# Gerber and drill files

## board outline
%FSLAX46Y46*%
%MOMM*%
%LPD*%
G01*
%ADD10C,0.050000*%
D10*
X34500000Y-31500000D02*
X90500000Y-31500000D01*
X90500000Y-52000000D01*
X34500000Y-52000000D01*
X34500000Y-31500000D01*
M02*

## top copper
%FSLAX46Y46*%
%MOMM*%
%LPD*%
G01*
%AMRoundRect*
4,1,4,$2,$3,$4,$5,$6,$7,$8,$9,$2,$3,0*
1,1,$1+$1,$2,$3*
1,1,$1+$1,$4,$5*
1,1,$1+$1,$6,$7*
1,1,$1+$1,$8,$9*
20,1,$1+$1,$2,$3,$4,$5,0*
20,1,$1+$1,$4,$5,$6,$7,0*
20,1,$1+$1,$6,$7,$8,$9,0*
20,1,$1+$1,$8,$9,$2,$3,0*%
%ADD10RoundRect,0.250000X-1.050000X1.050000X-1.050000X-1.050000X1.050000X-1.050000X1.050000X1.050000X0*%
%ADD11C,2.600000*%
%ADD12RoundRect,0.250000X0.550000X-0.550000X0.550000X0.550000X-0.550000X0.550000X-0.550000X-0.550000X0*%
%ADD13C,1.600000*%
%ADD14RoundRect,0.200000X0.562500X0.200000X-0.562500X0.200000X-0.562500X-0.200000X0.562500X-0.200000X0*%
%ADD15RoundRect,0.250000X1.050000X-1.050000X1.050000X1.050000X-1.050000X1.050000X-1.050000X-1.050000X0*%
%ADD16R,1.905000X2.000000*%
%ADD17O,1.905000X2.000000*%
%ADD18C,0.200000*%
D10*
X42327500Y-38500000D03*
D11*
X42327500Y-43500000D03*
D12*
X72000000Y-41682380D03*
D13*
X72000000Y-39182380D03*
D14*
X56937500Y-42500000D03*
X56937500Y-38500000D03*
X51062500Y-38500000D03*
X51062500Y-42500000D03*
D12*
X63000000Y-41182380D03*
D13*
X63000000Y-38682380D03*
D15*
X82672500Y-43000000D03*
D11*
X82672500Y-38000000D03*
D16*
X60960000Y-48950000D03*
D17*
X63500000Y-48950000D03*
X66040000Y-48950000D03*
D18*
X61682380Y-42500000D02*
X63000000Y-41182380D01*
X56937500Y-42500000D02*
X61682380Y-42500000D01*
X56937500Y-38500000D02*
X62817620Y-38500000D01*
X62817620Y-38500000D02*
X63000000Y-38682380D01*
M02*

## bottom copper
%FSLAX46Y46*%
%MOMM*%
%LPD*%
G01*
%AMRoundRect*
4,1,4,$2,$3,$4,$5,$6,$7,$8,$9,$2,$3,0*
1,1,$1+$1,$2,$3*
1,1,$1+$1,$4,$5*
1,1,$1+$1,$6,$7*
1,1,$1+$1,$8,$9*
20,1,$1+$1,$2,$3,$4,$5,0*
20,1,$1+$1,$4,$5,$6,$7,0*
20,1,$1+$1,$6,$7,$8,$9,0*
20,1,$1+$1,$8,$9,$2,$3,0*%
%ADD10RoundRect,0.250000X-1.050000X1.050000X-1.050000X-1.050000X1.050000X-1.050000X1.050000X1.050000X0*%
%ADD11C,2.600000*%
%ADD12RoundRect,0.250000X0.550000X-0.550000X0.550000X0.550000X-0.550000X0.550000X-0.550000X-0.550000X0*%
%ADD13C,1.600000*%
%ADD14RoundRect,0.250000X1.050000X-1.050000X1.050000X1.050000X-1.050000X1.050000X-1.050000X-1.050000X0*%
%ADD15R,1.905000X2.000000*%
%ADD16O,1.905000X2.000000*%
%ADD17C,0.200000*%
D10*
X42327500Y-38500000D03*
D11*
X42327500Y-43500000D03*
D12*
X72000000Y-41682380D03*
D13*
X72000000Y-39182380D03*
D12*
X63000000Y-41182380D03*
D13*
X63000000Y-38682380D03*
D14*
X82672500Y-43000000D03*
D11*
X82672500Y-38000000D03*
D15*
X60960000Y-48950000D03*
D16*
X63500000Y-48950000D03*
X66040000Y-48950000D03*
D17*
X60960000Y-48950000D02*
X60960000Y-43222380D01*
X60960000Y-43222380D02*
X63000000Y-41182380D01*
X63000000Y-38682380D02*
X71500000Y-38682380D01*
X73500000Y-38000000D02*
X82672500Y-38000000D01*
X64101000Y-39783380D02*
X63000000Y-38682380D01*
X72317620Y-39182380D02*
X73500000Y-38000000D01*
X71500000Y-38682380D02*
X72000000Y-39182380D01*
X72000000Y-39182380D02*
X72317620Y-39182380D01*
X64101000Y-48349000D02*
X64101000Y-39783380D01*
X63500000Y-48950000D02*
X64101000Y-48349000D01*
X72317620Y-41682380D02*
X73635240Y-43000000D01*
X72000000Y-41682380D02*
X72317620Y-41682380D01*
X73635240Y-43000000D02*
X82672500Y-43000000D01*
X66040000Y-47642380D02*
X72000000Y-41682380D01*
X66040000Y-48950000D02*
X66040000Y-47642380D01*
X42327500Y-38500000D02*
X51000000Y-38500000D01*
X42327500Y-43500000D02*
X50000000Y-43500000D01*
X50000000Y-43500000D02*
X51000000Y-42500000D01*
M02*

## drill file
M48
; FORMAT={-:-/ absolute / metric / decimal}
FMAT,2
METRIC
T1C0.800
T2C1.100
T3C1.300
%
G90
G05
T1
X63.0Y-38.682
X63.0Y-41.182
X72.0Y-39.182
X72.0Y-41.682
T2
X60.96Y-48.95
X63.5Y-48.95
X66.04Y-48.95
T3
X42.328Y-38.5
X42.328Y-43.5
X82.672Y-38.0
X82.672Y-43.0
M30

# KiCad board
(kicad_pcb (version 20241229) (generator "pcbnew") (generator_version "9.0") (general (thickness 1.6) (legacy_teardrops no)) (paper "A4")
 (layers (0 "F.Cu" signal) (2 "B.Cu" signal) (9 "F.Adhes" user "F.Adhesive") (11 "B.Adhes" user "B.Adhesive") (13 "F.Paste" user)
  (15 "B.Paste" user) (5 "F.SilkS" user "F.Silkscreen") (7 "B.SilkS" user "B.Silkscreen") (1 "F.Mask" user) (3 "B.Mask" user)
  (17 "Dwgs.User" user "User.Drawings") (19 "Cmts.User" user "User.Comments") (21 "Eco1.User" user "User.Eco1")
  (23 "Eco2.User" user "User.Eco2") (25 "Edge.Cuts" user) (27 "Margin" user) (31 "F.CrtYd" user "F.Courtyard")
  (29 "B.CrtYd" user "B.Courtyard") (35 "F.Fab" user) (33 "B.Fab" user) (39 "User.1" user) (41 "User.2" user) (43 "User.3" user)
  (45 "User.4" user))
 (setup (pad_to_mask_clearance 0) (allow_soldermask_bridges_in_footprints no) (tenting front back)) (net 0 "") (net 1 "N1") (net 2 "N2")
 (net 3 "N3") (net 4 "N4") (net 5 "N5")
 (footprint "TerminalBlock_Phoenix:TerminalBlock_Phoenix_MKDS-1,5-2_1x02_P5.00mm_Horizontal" (layer "F.Cu") (at 42.3275 38.5 -90)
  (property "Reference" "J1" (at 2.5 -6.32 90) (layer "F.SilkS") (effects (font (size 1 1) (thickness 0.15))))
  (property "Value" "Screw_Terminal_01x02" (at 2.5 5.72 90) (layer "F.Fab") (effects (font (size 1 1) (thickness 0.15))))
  (pad "1" thru_hole roundrect (at 0 0 270) (size 2.6 2.6) (drill 1.3) (layers "*.Cu" "*.Mask") (remove_unused_layers no)
   (roundrect_rratio 0.096154) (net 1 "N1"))
  (pad "2" thru_hole circle (at 5 0 270) (size 2.6 2.6) (drill 1.3) (layers "*.Cu" "*.Mask") (remove_unused_layers no) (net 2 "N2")))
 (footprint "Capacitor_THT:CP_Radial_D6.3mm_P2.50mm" (layer "F.Cu") (at 72 41.68238 90)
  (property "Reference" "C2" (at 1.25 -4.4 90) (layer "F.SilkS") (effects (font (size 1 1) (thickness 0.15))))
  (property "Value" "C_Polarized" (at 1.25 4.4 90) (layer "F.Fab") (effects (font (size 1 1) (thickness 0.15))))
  (pad "1" thru_hole roundrect (at 0 0 90) (size 1.6 1.6) (drill 0.8) (layers "*.Cu" "*.Mask") (remove_unused_layers no)
   (roundrect_rratio 0.15625) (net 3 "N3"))
  (pad "2" thru_hole circle (at 2.5 0 90) (size 1.6 1.6) (drill 0.8) (layers "*.Cu" "*.Mask") (remove_unused_layers no) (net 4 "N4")))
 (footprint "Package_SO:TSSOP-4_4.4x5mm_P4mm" (layer "F.Cu") (at 54 40.5 180)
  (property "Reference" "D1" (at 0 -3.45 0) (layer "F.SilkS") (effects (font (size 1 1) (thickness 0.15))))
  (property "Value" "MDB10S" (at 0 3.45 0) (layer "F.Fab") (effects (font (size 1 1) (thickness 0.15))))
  (pad "1" smd roundrect (at -2.9375 -2 180) (size 1.525 0.8) (layers "F.Cu" "F.Mask" "F.Paste") (roundrect_rratio 0.25) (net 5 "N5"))
  (pad "2" smd roundrect (at -2.9375 2 180) (size 1.525 0.8) (layers "F.Cu" "F.Mask" "F.Paste") (roundrect_rratio 0.25) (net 4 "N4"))
  (pad "3" smd roundrect (at 2.9375 2 180) (size 1.525 0.8) (layers "F.Cu" "F.Mask" "F.Paste") (roundrect_rratio 0.25) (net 1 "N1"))
  (pad "4" smd roundrect (at 2.9375 -2 180) (size 1.525 0.8) (layers "F.Cu" "F.Mask" "F.Paste") (roundrect_rratio 0.25) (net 2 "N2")))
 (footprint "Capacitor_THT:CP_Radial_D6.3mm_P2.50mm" (layer "F.Cu") (at 63 41.18238 90)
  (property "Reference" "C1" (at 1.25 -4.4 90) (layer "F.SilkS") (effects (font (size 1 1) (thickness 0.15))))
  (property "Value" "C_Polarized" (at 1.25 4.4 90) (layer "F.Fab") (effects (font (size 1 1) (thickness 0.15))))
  (pad "1" thru_hole roundrect (at 0 0 90) (size 1.6 1.6) (drill 0.8) (layers "*.Cu" "*.Mask") (remove_unused_layers no)
   (roundrect_rratio 0.15625) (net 5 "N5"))
  (pad "2" thru_hole circle (at 2.5 0 90) (size 1.6 1.6) (drill 0.8) (layers "*.Cu" "*.Mask") (remove_unused_layers no) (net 4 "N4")))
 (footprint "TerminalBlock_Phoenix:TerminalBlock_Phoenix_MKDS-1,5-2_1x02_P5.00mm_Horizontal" (layer "F.Cu") (at 82.6725 43 90)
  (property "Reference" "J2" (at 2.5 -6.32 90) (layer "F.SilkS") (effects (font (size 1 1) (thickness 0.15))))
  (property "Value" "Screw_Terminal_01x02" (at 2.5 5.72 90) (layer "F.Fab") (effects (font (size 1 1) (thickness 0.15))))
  (pad "1" thru_hole roundrect (at 0 0 90) (size 2.6 2.6) (drill 1.3) (layers "*.Cu" "*.Mask") (remove_unused_layers no)
   (roundrect_rratio 0.096154) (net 3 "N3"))
  (pad "2" thru_hole circle (at 5 0 90) (size 2.6 2.6) (drill 1.3) (layers "*.Cu" "*.Mask") (remove_unused_layers no) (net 4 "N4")))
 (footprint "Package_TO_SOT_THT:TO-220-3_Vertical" (layer "F.Cu") (at 60.96 48.95)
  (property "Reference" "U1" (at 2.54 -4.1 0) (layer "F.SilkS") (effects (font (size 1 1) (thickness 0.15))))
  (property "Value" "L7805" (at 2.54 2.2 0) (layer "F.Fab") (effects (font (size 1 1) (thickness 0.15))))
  (pad "1" thru_hole rect (at 0 0) (size 1.905 2) (drill 1.1) (layers "*.Cu" "*.Mask") (remove_unused_layers no) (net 5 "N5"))
  (pad "2" thru_hole oval (at 2.54 0) (size 1.905 2) (drill 1.1) (layers "*.Cu" "*.Mask") (remove_unused_layers no) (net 4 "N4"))
  (pad "3" thru_hole oval (at 5.08 0) (size 1.905 2) (drill 1.1) (layers "*.Cu" "*.Mask") (remove_unused_layers no) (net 3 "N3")))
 (gr_rect (start 34.5 31.5) (end 90.5 52) (stroke (width 0.05) (type default)) (fill no) (layer "Edge.Cuts"))
 (segment (start 61.68238 42.5) (end 63 41.18238) (width 0.2) (layer "F.Cu") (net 5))
 (segment (start 56.9375 42.5) (end 61.68238 42.5) (width 0.2) (layer "F.Cu") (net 5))
 (segment (start 60.96 48.95) (end 60.96 43.22238) (width 0.2) (layer "B.Cu") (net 5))
 (segment (start 60.96 43.22238) (end 63 41.18238) (width 0.2) (layer "B.Cu") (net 5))
 (segment (start 56.9375 38.5) (end 62.81762 38.5) (width 0.2) (layer "F.Cu") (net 4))
 (segment (start 62.81762 38.5) (end 63 38.68238) (width 0.2) (layer "F.Cu") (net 4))
 (segment (start 63 38.68238) (end 71.5 38.68238) (width 0.2) (layer "B.Cu") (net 4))
 (segment (start 73.5 38) (end 82.6725 38) (width 0.2) (layer "B.Cu") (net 4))
 (segment (start 64.101 39.78338) (end 63 38.68238) (width 0.2) (layer "B.Cu") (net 4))
 (segment (start 72.31762 39.18238) (end 73.5 38) (width 0.2) (layer "B.Cu") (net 4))
 (segment (start 71.5 38.68238) (end 72 39.18238) (width 0.2) (layer "B.Cu") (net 4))
 (segment (start 72 39.18238) (end 72.31762 39.18238) (width 0.2) (layer "B.Cu") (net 4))
 (segment (start 64.101 48.349) (end 64.101 39.78338) (width 0.2) (layer "B.Cu") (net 4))
 (segment (start 63.5 48.95) (end 64.101 48.349) (width 0.2) (layer "B.Cu") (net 4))
 (segment (start 72.31762 41.68238) (end 73.63524 43) (width 0.2) (layer "B.Cu") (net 3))
 (segment (start 72 41.68238) (end 72.31762 41.68238) (width 0.2) (layer "B.Cu") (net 3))
 (segment (start 73.63524 43) (end 82.6725 43) (width 0.2) (layer "B.Cu") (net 3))
 (segment (start 66.04 47.64238) (end 72 41.68238) (width 0.2) (layer "B.Cu") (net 3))
 (segment (start 66.04 48.95) (end 66.04 47.64238) (width 0.2) (layer "B.Cu") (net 3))
 (segment (start 42.3275 38.5) (end 51 38.5) (width 0.2) (layer "B.Cu") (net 1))
 (segment (start 42.3275 43.5) (end 50 43.5) (width 0.2) (layer "B.Cu") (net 2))
 (segment (start 50 43.5) (end 51 42.5) (width 0.2) (layer "B.Cu") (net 2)))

